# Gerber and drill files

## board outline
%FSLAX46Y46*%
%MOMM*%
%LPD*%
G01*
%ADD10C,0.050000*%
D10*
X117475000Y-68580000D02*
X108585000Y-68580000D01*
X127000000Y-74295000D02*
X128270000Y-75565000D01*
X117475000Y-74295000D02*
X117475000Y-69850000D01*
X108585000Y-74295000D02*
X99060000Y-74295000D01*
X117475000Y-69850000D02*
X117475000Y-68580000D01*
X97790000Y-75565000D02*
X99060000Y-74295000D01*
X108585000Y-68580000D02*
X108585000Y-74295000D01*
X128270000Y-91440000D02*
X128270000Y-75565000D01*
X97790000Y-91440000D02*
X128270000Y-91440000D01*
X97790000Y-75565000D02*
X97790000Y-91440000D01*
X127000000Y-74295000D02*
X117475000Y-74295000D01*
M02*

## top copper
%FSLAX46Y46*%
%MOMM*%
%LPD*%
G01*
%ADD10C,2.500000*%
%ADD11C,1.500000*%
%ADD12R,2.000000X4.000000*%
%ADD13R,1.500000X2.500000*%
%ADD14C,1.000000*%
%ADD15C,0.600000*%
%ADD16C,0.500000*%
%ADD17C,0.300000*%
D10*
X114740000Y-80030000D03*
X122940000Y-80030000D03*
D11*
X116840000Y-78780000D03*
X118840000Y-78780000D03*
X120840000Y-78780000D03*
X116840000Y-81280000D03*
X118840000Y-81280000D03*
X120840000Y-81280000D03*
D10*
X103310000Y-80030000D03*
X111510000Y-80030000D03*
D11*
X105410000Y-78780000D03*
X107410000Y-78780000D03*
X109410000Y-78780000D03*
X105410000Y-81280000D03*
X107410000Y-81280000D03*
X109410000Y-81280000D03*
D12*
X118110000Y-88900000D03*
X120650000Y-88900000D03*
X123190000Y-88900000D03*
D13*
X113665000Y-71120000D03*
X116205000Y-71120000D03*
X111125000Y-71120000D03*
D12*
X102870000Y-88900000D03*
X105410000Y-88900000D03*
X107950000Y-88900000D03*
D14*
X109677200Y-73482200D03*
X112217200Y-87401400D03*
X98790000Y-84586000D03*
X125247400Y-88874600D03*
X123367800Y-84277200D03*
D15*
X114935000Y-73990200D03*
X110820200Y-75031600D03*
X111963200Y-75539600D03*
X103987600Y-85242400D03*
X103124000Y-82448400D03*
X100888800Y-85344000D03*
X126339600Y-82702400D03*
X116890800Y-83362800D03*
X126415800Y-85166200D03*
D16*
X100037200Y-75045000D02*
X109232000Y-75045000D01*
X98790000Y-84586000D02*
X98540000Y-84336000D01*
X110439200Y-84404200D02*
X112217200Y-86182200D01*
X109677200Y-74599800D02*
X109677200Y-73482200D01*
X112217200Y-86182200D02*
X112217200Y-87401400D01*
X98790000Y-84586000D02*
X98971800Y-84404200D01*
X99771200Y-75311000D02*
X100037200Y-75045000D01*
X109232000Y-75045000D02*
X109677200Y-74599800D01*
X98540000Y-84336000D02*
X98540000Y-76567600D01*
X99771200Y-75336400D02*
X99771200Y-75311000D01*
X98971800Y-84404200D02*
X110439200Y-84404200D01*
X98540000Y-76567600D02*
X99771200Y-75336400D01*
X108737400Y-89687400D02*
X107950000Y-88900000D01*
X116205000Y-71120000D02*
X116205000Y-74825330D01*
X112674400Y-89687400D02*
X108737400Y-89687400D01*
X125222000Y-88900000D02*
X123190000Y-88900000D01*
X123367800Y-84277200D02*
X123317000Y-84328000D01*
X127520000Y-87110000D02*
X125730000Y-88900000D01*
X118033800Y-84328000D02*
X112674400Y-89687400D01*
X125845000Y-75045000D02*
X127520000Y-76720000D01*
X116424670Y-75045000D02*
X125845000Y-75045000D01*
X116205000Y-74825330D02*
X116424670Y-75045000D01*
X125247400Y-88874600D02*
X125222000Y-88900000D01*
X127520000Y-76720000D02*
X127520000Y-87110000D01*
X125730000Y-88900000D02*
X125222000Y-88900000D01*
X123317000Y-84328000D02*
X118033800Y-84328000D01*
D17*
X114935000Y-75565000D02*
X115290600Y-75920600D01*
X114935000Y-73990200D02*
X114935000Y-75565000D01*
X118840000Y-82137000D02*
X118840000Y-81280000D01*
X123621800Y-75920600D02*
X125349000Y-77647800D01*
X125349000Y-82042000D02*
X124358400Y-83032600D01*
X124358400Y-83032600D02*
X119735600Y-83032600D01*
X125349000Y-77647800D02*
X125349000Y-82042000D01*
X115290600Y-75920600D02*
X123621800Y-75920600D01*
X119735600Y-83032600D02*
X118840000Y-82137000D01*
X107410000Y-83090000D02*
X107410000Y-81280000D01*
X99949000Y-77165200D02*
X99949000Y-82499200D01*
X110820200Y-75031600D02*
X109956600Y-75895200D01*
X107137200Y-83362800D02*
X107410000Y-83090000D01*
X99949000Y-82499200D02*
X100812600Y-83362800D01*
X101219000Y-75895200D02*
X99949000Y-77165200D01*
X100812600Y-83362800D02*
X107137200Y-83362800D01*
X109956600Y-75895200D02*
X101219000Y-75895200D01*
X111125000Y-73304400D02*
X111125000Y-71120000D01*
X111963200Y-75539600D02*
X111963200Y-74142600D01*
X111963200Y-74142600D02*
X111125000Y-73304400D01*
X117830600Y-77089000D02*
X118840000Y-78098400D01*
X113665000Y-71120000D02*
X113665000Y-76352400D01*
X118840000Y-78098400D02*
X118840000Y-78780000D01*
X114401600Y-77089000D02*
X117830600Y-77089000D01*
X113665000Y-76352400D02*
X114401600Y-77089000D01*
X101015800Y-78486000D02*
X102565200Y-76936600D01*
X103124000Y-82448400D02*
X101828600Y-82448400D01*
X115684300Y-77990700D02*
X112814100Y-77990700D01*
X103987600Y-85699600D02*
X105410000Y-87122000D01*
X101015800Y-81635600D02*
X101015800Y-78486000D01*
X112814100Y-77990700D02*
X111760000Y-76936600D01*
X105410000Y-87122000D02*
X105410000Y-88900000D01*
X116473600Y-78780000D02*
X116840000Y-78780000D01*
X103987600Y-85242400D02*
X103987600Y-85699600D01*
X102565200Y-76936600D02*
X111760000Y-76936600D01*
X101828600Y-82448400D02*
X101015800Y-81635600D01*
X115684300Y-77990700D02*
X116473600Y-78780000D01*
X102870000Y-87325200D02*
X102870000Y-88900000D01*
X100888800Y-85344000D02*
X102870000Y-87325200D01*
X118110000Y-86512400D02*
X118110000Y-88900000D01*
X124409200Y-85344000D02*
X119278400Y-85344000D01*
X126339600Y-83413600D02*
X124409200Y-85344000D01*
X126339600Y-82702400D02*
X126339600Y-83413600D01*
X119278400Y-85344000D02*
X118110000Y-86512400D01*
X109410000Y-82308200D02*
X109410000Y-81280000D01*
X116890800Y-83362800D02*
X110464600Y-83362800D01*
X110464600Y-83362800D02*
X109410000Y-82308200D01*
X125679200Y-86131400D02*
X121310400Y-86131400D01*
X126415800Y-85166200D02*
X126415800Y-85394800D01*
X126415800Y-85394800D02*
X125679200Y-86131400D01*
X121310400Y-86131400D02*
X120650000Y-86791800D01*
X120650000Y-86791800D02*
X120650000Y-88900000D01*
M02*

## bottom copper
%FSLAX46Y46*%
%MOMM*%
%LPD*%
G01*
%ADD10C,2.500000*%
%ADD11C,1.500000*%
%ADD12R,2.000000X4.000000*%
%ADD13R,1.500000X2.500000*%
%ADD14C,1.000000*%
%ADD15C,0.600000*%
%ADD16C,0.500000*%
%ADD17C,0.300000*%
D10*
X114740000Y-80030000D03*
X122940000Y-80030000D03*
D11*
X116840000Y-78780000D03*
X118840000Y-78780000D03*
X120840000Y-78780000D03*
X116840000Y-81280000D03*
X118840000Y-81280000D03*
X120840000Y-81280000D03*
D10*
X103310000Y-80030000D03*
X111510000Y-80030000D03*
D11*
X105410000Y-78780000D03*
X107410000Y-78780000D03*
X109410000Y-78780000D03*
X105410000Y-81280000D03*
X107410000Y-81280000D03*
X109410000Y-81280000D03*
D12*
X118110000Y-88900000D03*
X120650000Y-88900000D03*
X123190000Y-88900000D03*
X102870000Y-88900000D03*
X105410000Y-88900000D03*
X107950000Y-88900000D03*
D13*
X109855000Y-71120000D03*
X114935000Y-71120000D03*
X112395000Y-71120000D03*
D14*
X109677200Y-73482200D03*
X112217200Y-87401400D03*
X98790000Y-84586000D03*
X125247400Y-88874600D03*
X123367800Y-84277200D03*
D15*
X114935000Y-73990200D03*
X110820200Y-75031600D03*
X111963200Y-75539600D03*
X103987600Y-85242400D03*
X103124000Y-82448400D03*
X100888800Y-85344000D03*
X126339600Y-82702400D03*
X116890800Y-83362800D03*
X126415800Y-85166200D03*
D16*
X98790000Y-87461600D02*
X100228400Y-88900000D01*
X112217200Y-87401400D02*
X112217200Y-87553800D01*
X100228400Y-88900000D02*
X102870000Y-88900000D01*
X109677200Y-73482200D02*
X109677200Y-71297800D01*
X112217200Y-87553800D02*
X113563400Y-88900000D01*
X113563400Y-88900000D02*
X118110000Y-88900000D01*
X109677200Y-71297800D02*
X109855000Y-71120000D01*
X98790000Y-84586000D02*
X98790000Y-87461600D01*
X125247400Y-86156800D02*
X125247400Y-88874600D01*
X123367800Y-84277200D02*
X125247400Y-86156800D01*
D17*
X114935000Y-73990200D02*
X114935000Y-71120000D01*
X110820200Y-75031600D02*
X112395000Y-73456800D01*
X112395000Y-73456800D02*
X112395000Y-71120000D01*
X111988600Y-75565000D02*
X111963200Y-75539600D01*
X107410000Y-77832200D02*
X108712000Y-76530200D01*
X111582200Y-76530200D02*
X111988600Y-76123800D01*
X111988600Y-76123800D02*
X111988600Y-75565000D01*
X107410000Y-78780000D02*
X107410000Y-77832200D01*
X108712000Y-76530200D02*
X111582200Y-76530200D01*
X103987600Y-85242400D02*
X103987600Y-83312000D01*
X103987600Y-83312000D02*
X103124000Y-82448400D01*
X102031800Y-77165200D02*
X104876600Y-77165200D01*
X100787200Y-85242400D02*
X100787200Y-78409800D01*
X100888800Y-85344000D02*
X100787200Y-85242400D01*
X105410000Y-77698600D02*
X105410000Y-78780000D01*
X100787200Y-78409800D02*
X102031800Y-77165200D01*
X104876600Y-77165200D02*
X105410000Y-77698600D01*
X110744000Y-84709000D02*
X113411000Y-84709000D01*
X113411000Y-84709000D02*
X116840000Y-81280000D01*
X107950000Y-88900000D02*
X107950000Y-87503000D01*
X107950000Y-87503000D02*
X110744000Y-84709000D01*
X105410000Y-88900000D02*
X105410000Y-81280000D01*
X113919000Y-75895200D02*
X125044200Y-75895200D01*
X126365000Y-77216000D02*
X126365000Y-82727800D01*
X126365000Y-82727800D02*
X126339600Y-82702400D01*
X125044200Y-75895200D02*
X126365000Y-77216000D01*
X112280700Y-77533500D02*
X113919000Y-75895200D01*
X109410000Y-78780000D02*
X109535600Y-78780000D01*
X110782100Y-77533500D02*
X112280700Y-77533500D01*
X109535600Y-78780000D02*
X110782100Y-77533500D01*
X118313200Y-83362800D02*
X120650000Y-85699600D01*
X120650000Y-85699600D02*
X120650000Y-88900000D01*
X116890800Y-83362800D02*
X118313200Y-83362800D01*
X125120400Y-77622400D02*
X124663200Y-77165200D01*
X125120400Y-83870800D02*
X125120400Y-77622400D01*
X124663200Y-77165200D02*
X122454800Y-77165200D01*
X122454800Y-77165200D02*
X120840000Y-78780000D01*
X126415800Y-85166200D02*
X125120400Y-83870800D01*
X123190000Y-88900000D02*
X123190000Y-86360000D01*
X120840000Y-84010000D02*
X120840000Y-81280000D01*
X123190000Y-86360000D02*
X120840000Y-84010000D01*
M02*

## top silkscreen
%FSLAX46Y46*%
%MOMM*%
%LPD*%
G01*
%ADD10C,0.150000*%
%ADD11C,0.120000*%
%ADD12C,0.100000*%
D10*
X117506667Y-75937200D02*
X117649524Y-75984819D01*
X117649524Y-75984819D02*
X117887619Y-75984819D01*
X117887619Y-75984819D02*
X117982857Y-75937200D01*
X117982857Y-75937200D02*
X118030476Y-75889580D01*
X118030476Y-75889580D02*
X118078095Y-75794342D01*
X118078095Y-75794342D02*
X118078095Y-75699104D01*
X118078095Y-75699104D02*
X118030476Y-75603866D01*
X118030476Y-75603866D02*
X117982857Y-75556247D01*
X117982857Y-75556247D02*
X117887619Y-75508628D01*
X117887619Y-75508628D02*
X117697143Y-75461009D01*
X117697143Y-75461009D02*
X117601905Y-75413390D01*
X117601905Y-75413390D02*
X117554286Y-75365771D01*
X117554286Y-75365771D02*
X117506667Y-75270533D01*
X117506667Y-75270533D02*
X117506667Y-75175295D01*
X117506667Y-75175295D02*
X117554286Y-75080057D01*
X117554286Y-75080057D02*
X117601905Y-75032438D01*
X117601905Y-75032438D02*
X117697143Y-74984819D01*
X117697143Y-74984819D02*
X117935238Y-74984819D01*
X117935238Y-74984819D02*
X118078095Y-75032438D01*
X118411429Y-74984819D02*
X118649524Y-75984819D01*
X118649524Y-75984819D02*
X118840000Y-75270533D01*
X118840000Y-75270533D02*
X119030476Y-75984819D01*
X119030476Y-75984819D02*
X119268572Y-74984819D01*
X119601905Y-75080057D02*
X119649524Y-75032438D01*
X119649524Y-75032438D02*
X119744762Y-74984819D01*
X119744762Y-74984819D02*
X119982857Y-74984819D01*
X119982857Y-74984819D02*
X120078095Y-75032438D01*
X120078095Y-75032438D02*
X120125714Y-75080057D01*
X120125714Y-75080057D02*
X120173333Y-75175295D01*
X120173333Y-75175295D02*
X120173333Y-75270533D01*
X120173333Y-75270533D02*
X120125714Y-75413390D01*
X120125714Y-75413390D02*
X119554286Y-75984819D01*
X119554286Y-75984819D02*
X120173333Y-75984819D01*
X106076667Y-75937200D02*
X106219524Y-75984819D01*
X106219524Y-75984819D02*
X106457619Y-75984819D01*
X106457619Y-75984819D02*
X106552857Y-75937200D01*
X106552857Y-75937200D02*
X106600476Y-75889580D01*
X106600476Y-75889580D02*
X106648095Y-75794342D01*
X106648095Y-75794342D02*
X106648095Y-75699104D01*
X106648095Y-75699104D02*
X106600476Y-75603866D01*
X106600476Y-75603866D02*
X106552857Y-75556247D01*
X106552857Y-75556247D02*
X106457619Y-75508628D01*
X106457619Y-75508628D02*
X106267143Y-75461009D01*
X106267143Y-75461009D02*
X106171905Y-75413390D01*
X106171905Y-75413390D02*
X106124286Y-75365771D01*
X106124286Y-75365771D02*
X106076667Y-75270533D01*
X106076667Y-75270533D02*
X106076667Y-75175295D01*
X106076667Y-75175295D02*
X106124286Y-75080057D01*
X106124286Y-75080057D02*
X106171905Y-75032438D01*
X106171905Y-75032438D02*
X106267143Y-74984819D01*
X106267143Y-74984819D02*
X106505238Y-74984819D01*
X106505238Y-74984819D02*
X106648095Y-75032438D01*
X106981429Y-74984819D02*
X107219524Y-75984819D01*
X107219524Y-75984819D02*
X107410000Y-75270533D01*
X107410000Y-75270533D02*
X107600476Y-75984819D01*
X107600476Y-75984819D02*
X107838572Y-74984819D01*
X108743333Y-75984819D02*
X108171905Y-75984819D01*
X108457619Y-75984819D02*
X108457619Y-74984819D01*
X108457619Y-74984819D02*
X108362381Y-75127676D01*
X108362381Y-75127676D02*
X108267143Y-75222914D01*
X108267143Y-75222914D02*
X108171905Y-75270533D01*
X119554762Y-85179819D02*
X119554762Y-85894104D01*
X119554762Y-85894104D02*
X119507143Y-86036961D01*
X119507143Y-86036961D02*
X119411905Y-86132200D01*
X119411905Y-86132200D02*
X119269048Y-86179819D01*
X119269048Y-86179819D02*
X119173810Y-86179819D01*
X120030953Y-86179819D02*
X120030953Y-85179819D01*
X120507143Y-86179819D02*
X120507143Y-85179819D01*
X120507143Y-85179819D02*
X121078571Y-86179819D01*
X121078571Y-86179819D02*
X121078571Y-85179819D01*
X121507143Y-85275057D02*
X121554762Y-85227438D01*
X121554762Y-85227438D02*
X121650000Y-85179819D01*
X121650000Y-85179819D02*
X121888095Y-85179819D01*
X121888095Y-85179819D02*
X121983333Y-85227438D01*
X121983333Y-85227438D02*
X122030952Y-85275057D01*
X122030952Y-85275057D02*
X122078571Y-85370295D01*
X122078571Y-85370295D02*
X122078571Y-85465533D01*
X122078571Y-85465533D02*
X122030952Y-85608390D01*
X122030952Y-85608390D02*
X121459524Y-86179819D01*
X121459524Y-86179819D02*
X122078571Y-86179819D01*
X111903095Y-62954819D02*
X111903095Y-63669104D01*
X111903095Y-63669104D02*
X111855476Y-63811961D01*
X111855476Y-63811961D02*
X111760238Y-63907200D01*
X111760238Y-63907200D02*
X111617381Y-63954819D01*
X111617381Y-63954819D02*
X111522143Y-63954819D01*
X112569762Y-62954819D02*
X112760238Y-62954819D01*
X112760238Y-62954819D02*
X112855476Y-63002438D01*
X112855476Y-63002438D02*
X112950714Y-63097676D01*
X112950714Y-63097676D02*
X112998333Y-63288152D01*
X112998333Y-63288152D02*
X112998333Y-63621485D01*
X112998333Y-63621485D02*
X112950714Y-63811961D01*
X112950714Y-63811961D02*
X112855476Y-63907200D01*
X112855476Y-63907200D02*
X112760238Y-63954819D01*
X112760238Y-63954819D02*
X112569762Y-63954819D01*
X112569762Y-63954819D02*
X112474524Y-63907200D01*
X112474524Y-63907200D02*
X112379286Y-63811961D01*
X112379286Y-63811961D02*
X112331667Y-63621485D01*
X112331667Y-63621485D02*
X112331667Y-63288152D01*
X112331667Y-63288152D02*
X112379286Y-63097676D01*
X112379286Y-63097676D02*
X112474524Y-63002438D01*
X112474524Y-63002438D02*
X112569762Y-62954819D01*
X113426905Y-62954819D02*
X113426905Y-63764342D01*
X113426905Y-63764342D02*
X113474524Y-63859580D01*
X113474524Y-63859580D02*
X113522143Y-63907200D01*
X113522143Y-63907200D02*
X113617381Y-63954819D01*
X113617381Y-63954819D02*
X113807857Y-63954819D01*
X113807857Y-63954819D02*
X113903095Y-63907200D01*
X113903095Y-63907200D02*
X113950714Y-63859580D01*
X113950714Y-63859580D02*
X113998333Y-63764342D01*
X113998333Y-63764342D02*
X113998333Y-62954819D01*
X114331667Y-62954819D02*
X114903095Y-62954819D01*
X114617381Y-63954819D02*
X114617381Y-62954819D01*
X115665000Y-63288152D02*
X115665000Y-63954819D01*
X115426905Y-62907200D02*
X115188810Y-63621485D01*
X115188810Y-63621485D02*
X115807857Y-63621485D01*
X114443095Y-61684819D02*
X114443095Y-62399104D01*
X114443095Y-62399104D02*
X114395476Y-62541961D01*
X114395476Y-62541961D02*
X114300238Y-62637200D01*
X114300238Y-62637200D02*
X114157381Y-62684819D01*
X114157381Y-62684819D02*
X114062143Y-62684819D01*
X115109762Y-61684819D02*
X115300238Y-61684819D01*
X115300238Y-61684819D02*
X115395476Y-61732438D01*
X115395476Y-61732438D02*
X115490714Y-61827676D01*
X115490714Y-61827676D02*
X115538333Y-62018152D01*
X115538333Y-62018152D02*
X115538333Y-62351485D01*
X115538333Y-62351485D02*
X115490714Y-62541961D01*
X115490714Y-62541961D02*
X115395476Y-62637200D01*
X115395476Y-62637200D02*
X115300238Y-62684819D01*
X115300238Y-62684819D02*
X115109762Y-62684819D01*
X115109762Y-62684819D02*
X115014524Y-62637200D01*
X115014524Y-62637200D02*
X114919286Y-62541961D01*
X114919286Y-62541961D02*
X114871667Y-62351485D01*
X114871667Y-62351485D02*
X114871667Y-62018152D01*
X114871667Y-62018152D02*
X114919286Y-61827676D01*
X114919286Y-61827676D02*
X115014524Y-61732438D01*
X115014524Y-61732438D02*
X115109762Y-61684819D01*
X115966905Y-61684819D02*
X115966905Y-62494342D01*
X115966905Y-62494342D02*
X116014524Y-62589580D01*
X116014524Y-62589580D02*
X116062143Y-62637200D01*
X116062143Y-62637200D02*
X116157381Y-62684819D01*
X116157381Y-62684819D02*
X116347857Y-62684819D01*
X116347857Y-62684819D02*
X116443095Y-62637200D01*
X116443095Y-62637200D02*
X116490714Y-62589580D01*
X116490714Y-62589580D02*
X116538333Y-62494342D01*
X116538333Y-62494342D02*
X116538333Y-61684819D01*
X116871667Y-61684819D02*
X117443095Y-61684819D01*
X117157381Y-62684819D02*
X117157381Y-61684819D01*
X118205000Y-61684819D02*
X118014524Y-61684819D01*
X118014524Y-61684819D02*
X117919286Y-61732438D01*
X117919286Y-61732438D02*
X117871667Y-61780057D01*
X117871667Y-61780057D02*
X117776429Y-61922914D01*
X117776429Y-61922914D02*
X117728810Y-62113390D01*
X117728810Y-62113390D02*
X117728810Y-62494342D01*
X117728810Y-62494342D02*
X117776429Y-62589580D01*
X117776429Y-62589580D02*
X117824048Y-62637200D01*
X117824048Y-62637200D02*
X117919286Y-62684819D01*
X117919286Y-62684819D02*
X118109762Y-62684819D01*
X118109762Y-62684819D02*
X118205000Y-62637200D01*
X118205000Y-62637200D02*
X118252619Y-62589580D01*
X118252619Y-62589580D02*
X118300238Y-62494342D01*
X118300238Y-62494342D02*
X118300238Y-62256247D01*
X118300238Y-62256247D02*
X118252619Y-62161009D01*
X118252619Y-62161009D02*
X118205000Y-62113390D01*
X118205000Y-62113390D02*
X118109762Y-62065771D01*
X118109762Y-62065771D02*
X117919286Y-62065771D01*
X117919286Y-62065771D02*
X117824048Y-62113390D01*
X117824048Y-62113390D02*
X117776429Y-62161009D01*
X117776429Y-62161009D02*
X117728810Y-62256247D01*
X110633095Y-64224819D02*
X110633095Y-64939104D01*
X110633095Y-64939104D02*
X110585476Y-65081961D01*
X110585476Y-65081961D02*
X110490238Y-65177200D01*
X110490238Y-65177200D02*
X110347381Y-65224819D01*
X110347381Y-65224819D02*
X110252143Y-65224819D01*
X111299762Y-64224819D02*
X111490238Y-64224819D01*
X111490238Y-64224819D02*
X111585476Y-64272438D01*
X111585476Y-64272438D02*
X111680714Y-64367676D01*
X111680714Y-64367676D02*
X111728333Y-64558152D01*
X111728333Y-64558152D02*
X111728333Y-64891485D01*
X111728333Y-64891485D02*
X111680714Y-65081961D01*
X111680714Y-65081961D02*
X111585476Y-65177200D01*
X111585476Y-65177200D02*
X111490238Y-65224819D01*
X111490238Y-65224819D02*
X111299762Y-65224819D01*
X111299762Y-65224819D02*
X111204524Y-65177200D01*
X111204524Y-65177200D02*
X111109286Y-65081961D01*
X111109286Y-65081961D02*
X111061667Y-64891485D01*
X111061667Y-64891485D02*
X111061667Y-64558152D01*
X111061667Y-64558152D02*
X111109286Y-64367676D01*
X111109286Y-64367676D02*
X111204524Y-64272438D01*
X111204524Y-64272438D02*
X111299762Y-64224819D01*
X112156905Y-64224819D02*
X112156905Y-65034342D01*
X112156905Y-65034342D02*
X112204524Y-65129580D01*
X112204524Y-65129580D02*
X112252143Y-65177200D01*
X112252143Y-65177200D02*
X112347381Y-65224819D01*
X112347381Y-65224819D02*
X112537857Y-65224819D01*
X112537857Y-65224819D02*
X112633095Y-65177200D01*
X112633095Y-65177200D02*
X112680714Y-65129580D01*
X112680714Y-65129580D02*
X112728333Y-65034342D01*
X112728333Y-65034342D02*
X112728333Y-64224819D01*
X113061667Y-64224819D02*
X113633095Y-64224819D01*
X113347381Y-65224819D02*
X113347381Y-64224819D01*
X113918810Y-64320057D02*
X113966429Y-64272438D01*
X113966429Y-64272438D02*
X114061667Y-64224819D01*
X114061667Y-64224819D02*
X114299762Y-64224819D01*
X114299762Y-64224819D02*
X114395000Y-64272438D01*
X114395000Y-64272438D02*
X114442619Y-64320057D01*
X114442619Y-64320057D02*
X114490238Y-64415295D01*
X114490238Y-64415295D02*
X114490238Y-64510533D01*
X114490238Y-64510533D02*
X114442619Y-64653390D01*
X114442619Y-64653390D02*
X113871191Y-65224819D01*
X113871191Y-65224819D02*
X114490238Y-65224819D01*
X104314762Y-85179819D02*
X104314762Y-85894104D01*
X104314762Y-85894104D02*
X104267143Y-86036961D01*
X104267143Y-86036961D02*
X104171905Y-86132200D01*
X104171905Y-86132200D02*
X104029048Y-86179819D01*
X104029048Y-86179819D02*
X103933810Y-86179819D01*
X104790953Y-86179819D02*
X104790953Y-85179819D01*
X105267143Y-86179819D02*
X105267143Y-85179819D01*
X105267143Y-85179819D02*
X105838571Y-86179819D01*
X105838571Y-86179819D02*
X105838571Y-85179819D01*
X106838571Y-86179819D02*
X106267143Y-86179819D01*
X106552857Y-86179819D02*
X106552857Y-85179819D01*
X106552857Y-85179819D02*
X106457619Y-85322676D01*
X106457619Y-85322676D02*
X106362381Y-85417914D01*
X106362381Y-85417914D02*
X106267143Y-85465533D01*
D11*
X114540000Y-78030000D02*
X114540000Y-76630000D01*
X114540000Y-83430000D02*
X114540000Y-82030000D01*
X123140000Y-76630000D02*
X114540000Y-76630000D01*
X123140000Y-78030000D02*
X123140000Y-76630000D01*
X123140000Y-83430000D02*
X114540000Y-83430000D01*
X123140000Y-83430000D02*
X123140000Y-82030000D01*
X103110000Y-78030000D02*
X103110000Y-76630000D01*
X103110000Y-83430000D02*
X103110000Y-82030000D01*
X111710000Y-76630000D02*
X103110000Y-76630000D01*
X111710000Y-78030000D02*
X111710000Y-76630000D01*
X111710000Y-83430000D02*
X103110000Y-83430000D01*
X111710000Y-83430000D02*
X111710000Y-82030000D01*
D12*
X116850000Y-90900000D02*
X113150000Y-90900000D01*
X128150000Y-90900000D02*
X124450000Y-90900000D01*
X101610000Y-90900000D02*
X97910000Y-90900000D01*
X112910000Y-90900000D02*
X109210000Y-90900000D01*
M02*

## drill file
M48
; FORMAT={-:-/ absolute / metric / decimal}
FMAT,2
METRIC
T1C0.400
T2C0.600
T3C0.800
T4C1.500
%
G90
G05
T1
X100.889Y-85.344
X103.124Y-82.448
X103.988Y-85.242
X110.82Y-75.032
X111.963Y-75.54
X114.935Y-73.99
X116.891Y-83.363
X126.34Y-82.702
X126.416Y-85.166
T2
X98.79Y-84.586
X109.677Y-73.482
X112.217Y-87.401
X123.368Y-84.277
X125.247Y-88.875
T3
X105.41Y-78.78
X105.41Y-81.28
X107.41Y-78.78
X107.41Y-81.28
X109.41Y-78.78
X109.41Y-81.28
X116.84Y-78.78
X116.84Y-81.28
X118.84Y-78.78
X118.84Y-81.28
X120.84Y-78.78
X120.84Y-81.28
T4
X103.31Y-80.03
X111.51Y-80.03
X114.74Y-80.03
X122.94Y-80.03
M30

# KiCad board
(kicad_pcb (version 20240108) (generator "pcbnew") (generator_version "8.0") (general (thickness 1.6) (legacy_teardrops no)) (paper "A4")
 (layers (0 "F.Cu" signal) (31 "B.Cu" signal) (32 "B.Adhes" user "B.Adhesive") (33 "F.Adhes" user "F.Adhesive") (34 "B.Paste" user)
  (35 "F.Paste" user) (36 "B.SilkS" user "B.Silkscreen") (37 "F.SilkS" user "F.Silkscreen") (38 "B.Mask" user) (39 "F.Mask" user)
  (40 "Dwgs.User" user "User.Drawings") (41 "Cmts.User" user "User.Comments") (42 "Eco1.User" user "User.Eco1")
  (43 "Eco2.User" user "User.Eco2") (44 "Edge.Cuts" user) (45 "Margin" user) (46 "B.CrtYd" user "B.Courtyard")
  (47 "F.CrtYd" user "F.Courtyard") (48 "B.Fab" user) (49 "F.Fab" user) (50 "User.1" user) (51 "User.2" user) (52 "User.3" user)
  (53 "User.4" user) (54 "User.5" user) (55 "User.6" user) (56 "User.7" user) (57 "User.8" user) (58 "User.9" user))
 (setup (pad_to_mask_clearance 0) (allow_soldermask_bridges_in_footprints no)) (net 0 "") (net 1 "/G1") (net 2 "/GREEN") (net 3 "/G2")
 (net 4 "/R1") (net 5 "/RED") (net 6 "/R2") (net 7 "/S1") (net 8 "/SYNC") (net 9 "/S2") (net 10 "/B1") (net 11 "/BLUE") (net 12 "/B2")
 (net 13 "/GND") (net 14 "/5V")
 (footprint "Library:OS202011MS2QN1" (layer "F.Cu") (at 118.84 80.03)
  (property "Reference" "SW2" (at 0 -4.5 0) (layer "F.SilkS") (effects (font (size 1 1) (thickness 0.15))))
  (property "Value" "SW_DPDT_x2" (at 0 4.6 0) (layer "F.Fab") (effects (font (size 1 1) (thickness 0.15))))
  (fp_line (start -4.3 -2) (end -4.3 -3.4) (stroke (width 0.12) (type solid)) (layer "F.SilkS"))
  (fp_line (start -4.3 3.4) (end -4.3 2) (stroke (width 0.12) (type solid)) (layer "F.SilkS"))
  (fp_line (start 4.3 -3.4) (end -4.3 -3.4) (stroke (width 0.12) (type solid)) (layer "F.SilkS"))
  (fp_line (start 4.3 -2) (end 4.3 -3.4) (stroke (width 0.12) (type solid)) (layer "F.SilkS"))
  (fp_line (start 4.3 3.4) (end -4.3 3.4) (stroke (width 0.12) (type solid)) (layer "F.SilkS"))
  (fp_line (start 4.3 3.4) (end 4.3 2) (stroke (width 0.12) (type solid)) (layer "F.SilkS"))
  (pad "" thru_hole circle (at -4.1 0) (size 2.5 2.5) (drill 1.5) (layers "*.Cu" "*.Mask") (remove_unused_layers no))
  (pad "" thru_hole circle (at 4.1 0) (size 2.5 2.5) (drill 1.5) (layers "*.Cu" "*.Mask") (remove_unused_layers no))
  (pad "1" thru_hole circle (at -2 -1.25) (size 1.5 1.5) (drill 0.8) (layers "*.Cu" "*.Mask") (remove_unused_layers no) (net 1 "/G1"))
  (pad "2" thru_hole circle (at 0 -1.25) (size 1.5 1.5) (drill 0.8) (layers "*.Cu" "*.Mask") (remove_unused_layers no) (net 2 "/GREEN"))
  (pad "3" thru_hole circle (at 2 -1.25) (size 1.5 1.5) (drill 0.8) (layers "*.Cu" "*.Mask") (remove_unused_layers no) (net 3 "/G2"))
  (pad "4" thru_hole circle (at -2 1.25) (size 1.5 1.5) (drill 0.8) (layers "*.Cu" "*.Mask") (remove_unused_layers no) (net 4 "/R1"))
  (pad "5" thru_hole circle (at 0 1.25) (size 1.5 1.5) (drill 0.8) (layers "*.Cu" "*.Mask") (remove_unused_layers no) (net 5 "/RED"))
  (pad "6" thru_hole circle (at 2 1.25) (size 1.5 1.5) (drill 0.8) (layers "*.Cu" "*.Mask") (remove_unused_layers no) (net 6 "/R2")))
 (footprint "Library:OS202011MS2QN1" (layer "F.Cu") (at 107.41 80.03)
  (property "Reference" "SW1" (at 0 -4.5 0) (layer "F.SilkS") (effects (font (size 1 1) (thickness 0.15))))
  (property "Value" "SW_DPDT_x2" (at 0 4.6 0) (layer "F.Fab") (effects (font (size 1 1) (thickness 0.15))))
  (fp_line (start -4.3 -2) (end -4.3 -3.4) (stroke (width 0.12) (type solid)) (layer "F.SilkS"))
  (fp_line (start -4.3 3.4) (end -4.3 2) (stroke (width 0.12) (type solid)) (layer "F.SilkS"))
  (fp_line (start 4.3 -3.4) (end -4.3 -3.4) (stroke (width 0.12) (type solid)) (layer "F.SilkS"))
  (fp_line (start 4.3 -2) (end 4.3 -3.4) (stroke (width 0.12) (type solid)) (layer "F.SilkS"))
  (fp_line (start 4.3 3.4) (end -4.3 3.4) (stroke (width 0.12) (type solid)) (layer "F.SilkS"))
  (fp_line (start 4.3 3.4) (end 4.3 2) (stroke (width 0.12) (type solid)) (layer "F.SilkS"))
  (pad "" thru_hole circle (at -4.1 0) (size 2.5 2.5) (drill 1.5) (layers "*.Cu" "*.Mask") (remove_unused_layers no))
  (pad "" thru_hole circle (at 4.1 0) (size 2.5 2.5) (drill 1.5) (layers "*.Cu" "*.Mask") (remove_unused_layers no))
  (pad "1" thru_hole circle (at -2 -1.25) (size 1.5 1.5) (drill 0.8) (layers "*.Cu" "*.Mask") (remove_unused_layers no) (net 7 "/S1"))
  (pad "2" thru_hole circle (at 0 -1.25) (size 1.5 1.5) (drill 0.8) (layers "*.Cu" "*.Mask") (remove_unused_layers no) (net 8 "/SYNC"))
  (pad "3" thru_hole circle (at 2 -1.25) (size 1.5 1.5) (drill 0.8) (layers "*.Cu" "*.Mask") (remove_unused_layers no) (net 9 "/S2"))
  (pad "4" thru_hole circle (at -2 1.25) (size 1.5 1.5) (drill 0.8) (layers "*.Cu" "*.Mask") (remove_unused_layers no) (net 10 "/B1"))
  (pad "5" thru_hole circle (at 0 1.25) (size 1.5 1.5) (drill 0.8) (layers "*.Cu" "*.Mask") (remove_unused_layers no) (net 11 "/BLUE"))
  (pad "6" thru_hole circle (at 2 1.25) (size 1.5 1.5) (drill 0.8) (layers "*.Cu" "*.Mask") (remove_unused_layers no) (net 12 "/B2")))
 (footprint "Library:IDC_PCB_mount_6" (layer "F.Cu") (at 120.65 88.9)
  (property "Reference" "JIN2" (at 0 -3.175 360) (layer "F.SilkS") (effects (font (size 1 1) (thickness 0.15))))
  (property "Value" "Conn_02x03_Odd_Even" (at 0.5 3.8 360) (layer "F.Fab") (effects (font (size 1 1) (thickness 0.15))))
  (fp_line (start -3.8 2) (end -7.5 2) (stroke (width 0.1) (type default)) (layer "F.SilkS"))
  (fp_line (start 7.5 2) (end 3.8 2) (stroke (width 0.1) (type default)) (layer "F.SilkS"))
  (pad "1" smd rect (at -2.54 0) (size 2 4) (layers "B.Cu" "B.Mask") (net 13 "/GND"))
  (pad "2" smd rect (at -2.54 0) (size 2 4) (layers "F.Cu" "F.Mask") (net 9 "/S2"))
  (pad "3" smd rect (at 0 0) (size 2 4) (layers "B.Cu" "B.Mask") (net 12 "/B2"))
  (pad "4" smd rect (at 0 0) (size 2 4) (layers "F.Cu" "F.Mask") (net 3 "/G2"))
  (pad "5" smd rect (at 2.54 0) (size 2 4) (layers "B.Cu" "B.Mask") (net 6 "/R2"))
  (pad "6" smd rect (at 2.54 0) (size 2 4) (layers "F.Cu" "F.Mask") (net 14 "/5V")))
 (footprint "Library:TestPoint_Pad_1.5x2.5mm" (layer "F.Cu") (at 113.665 71.12)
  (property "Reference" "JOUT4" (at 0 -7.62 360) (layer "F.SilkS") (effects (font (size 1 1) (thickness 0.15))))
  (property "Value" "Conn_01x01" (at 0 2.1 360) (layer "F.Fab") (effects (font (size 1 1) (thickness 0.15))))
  (pad "1" smd rect (at 0 0) (size 1.5 2.5) (layers "F.Cu" "F.Mask") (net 2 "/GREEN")))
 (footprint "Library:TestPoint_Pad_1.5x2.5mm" (layer "F.Cu") (at 116.205 71.12)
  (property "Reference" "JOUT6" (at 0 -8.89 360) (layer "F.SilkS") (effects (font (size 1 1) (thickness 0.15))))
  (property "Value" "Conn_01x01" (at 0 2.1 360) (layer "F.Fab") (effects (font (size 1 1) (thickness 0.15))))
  (pad "1" smd rect (at 0 0) (size 1.5 2.5) (layers "F.Cu" "F.Mask") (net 14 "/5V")))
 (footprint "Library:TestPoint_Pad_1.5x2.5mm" (layer "F.Cu") (at 111.125 71.12)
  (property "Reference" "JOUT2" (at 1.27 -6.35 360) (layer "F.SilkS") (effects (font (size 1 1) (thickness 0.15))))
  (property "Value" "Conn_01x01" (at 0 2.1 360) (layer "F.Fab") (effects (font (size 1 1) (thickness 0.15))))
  (pad "1" smd rect (at 0 0) (size 1.5 2.5) (layers "F.Cu" "F.Mask") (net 8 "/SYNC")))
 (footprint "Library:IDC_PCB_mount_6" (layer "F.Cu") (at 105.41 88.9)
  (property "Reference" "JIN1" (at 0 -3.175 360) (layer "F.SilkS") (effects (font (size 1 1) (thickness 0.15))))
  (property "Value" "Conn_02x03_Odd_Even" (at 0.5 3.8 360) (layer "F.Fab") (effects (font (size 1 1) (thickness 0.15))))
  (fp_line (start -3.8 2) (end -7.5 2) (stroke (width 0.1) (type default)) (layer "F.SilkS"))
  (fp_line (start 7.5 2) (end 3.8 2) (stroke (width 0.1) (type default)) (layer "F.SilkS"))
  (pad "1" smd rect (at -2.54 0) (size 2 4) (layers "B.Cu" "B.Mask") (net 13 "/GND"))
  (pad "2" smd rect (at -2.54 0) (size 2 4) (layers "F.Cu" "F.Mask") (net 7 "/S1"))
  (pad "3" smd rect (at 0 0) (size 2 4) (layers "B.Cu" "B.Mask") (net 10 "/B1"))
  (pad "4" smd rect (at 0 0) (size 2 4) (layers "F.Cu" "F.Mask") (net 1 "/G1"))
  (pad "5" smd rect (at 2.54 0) (size 2 4) (layers "B.Cu" "B.Mask") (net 4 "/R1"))
  (pad "6" smd rect (at 2.54 0) (size 2 4) (layers "F.Cu" "F.Mask") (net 14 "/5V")))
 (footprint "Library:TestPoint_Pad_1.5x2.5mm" (layer "B.Cu") (at 109.855 71.12 180)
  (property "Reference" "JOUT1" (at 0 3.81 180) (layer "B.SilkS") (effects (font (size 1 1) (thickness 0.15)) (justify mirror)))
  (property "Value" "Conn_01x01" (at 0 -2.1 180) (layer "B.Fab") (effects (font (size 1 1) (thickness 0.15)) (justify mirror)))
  (pad "1" smd rect (at 0 0 180) (size 1.5 2.5) (layers "B.Cu" "B.Mask") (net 13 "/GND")))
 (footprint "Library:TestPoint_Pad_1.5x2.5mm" (layer "B.Cu") (at 114.935 71.12 180)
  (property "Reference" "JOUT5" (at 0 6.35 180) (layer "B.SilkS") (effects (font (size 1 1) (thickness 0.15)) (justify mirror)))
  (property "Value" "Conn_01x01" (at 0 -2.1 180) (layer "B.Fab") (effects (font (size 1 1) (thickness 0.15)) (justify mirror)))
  (pad "1" smd rect (at 0 0 180) (size 1.5 2.5) (layers "B.Cu" "B.Mask") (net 5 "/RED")))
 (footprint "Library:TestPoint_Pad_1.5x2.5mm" (layer "B.Cu") (at 112.395 71.12 180)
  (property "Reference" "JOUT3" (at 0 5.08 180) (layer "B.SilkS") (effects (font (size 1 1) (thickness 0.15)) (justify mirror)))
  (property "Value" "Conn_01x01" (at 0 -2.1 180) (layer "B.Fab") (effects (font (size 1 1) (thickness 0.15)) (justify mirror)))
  (pad "1" smd rect (at 0 0 180) (size 1.5 2.5) (layers "B.Cu" "B.Mask") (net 11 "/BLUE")))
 (gr_line (start 117.475 68.58) (end 108.585 68.58) (stroke (width 0.05) (type default)) (layer "Edge.Cuts"))
 (gr_line (start 127 74.295) (end 128.27 75.565) (stroke (width 0.05) (type default)) (layer "Edge.Cuts"))
 (gr_line (start 117.475 74.295) (end 117.475 69.85) (stroke (width 0.05) (type default)) (layer "Edge.Cuts"))
 (gr_line (start 108.585 74.295) (end 99.06 74.295) (stroke (width 0.05) (type default)) (layer "Edge.Cuts"))
 (gr_line (start 117.475 69.85) (end 117.475 68.58) (stroke (width 0.05) (type default)) (layer "Edge.Cuts"))
 (gr_line (start 97.79 75.565) (end 99.06 74.295) (stroke (width 0.05) (type default)) (layer "Edge.Cuts"))
 (gr_line (start 108.585 68.58) (end 108.585 74.295) (stroke (width 0.05) (type default)) (layer "Edge.Cuts"))
 (gr_line (start 128.27 91.44) (end 128.27 75.565) (stroke (width 0.05) (type default)) (layer "Edge.Cuts"))
 (gr_line (start 97.79 91.44) (end 128.27 91.44) (stroke (width 0.05) (type default)) (layer "Edge.Cuts"))
 (gr_line (start 97.79 75.565) (end 97.79 91.44) (stroke (width 0.05) (type default)) (layer "Edge.Cuts"))
 (gr_line (start 127 74.295) (end 117.475 74.295) (stroke (width 0.05) (type default)) (layer "Edge.Cuts"))
 (segment (start 100.0372 75.045) (end 109.232 75.045) (width 0.5) (layer "F.Cu") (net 13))
 (segment (start 98.79 84.586) (end 98.54 84.336) (width 0.5) (layer "F.Cu") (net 13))
 (segment (start 110.4392 84.4042) (end 112.2172 86.1822) (width 0.5) (layer "F.Cu") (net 13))
 (segment (start 109.6772 74.5998) (end 109.6772 73.4822) (width 0.5) (layer "F.Cu") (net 13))
 (segment (start 112.2172 86.1822) (end 112.2172 87.4014) (width 0.5) (layer "F.Cu") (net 13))
 (segment (start 98.79 84.586) (end 98.9718 84.4042) (width 0.5) (layer "F.Cu") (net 13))
 (segment (start 99.7712 75.311) (end 100.0372 75.045) (width 0.5) (layer "F.Cu") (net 13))
 (segment (start 109.232 75.045) (end 109.6772 74.5998) (width 0.5) (layer "F.Cu") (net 13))
 (segment (start 98.54 84.336) (end 98.54 76.5676) (width 0.5) (layer "F.Cu") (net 13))
 (segment (start 99.7712 75.3364) (end 99.7712 75.311) (width 0.5) (layer "F.Cu") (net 13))
 (segment (start 98.9718 84.4042) (end 110.4392 84.4042) (width 0.5) (layer "F.Cu") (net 13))
 (segment (start 98.54 76.5676) (end 99.7712 75.3364) (width 0.5) (layer "F.Cu") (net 13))
 (via (at 109.6772 73.4822) (size 1) (drill 0.6) (layers "F.Cu" "B.Cu") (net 13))
 (via (at 112.2172 87.4014) (size 1) (drill 0.6) (layers "F.Cu" "B.Cu") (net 13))
 (via (at 98.79 84.586) (size 1) (drill 0.6) (layers "F.Cu" "B.Cu") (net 13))
 (segment (start 98.79 87.4616) (end 100.2284 88.9) (width 0.5) (layer "B.Cu") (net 13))
 (segment (start 112.2172 87.4014) (end 112.2172 87.5538) (width 0.5) (layer "B.Cu") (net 13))
 (segment (start 100.2284 88.9) (end 102.87 88.9) (width 0.5) (layer "B.Cu") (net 13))
 (segment (start 109.6772 73.4822) (end 109.6772 71.2978) (width 0.5) (layer "B.Cu") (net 13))
 (segment (start 112.2172 87.5538) (end 113.5634 88.9) (width 0.5) (layer "B.Cu") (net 13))
 (segment (start 113.5634 88.9) (end 118.11 88.9) (width 0.5) (layer "B.Cu") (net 13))
 (segment (start 109.6772 71.2978) (end 109.855 71.12) (width 0.5) (layer "B.Cu") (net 13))
 (segment (start 98.79 84.586) (end 98.79 87.4616) (width 0.5) (layer "B.Cu") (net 13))
 (segment (start 108.7374 89.6874) (end 107.95 88.9) (width 0.5) (layer "F.Cu") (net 14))
 (segment (start 116.205 71.12) (end 116.205 74.82533) (width 0.5) (layer "F.Cu") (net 14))
 (segment (start 112.6744 89.6874) (end 108.7374 89.6874) (width 0.5) (layer "F.Cu") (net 14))
 (segment (start 125.222 88.9) (end 123.19 88.9) (width 0.5) (layer "F.Cu") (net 14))
 (segment (start 123.3678 84.2772) (end 123.317 84.328) (width 0.5) (layer "F.Cu") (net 14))
 (segment (start 127.52 87.11) (end 125.73 88.9) (width 0.5) (layer "F.Cu") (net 14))
 (segment (start 118.0338 84.328) (end 112.6744 89.6874) (width 0.5) (layer "F.Cu") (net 14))
 (segment (start 125.845 75.045) (end 127.52 76.72) (width 0.5) (layer "F.Cu") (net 14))
 (segment (start 116.42467 75.045) (end 125.845 75.045) (width 0.5) (layer "F.Cu") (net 14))
 (segment (start 116.205 74.82533) (end 116.42467 75.045) (width 0.5) (layer "F.Cu") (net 14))
 (segment (start 125.2474 88.8746) (end 125.222 88.9) (width 0.5) (layer "F.Cu") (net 14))
 (segment (start 127.52 76.72) (end 127.52 87.11) (width 0.5) (layer "F.Cu") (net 14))
 (segment (start 125.73 88.9) (end 125.222 88.9) (width 0.5) (layer "F.Cu") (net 14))
 (segment (start 123.317 84.328) (end 118.0338 84.328) (width 0.5) (layer "F.Cu") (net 14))
 (via (at 125.2474 88.8746) (size 1) (drill 0.6) (layers "F.Cu" "B.Cu") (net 14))
 (via (at 123.3678 84.2772) (size 1) (drill 0.6) (layers "F.Cu" "B.Cu") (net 14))
 (segment (start 125.2474 86.1568) (end 125.2474 88.8746) (width 0.5) (layer "B.Cu") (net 14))
 (segment (start 123.3678 84.2772) (end 125.2474 86.1568) (width 0.5) (layer "B.Cu") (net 14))
 (segment (start 114.935 75.565) (end 115.2906 75.9206) (width 0.3) (layer "F.Cu") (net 5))
 (segment (start 114.935 73.9902) (end 114.935 75.565) (width 0.3) (layer "F.Cu") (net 5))
 (segment (start 118.84 82.137) (end 118.84 81.28) (width 0.3) (layer "F.Cu") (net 5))
 (segment (start 123.6218 75.9206) (end 125.349 77.6478) (width 0.3) (layer "F.Cu") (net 5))
 (segment (start 125.349 82.042) (end 124.3584 83.0326) (width 0.3) (layer "F.Cu") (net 5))
 (segment (start 124.3584 83.0326) (end 119.7356 83.0326) (width 0.3) (layer "F.Cu") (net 5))
 (segment (start 125.349 77.6478) (end 125.349 82.042) (width 0.3) (layer "F.Cu") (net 5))
 (segment (start 115.2906 75.9206) (end 123.6218 75.9206) (width 0.3) (layer "F.Cu") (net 5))
 (segment (start 119.7356 83.0326) (end 118.84 82.137) (width 0.3) (layer "F.Cu") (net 5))
 (via (at 114.935 73.9902) (size 0.6) (drill 0.4) (layers "F.Cu" "B.Cu") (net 5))
 (segment (start 114.935 73.9902) (end 114.935 71.12) (width 0.3) (layer "B.Cu") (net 5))
 (segment (start 107.41 83.09) (end 107.41 81.28) (width 0.3) (layer "F.Cu") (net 11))
 (segment (start 99.949 77.1652) (end 99.949 82.4992) (width 0.3) (layer "F.Cu") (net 11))
 (segment (start 110.8202 75.0316) (end 109.9566 75.8952) (width 0.3) (layer "F.Cu") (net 11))
 (segment (start 107.1372 83.3628) (end 107.41 83.09) (width 0.3) (layer "F.Cu") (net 11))
 (segment (start 99.949 82.4992) (end 100.8126 83.3628) (width 0.3) (layer "F.Cu") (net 11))
 (segment (start 101.219 75.8952) (end 99.949 77.1652) (width 0.3) (layer "F.Cu") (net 11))
 (segment (start 100.8126 83.3628) (end 107.1372 83.3628) (width 0.3) (layer "F.Cu") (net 11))
 (segment (start 109.9566 75.8952) (end 101.219 75.8952) (width 0.3) (layer "F.Cu") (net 11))
 (via (at 110.8202 75.0316) (size 0.6) (drill 0.4) (layers "F.Cu" "B.Cu") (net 11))
 (segment (start 110.8202 75.0316) (end 112.395 73.4568) (width 0.3) (layer "B.Cu") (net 11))
 (segment (start 112.395 73.4568) (end 112.395 71.12) (width 0.3) (layer "B.Cu") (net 11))
 (segment (start 111.125 73.3044) (end 111.125 71.12) (width 0.3) (layer "F.Cu") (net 8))
 (segment (start 111.9632 75.5396) (end 111.9632 74.1426) (width 0.3) (layer "F.Cu") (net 8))
 (segment (start 111.9632 74.1426) (end 111.125 73.3044) (width 0.3) (layer "F.Cu") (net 8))
 (via (at 111.9632 75.5396) (size 0.6) (drill 0.4) (layers "F.Cu" "B.Cu") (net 8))
 (segment (start 111.9886 75.565) (end 111.9632 75.5396) (width 0.3) (layer "B.Cu") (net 8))
 (segment (start 107.41 77.8322) (end 108.712 76.5302) (width 0.3) (layer "B.Cu") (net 8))
 (segment (start 111.5822 76.5302) (end 111.9886 76.1238) (width 0.3) (layer "B.Cu") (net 8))
 (segment (start 111.9886 76.1238) (end 111.9886 75.565) (width 0.3) (layer "B.Cu") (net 8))
 (segment (start 107.41 78.78) (end 107.41 77.8322) (width 0.3) (layer "B.Cu") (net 8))
 (segment (start 108.712 76.5302) (end 111.5822 76.5302) (width 0.3) (layer "B.Cu") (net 8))
 (segment (start 117.8306 77.089) (end 118.84 78.0984) (width 0.3) (layer "F.Cu") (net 2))
 (segment (start 113.665 71.12) (end 113.665 76.3524) (width 0.3) (layer "F.Cu") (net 2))
 (segment (start 118.84 78.0984) (end 118.84 78.78) (width 0.3) (layer "F.Cu") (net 2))
 (segment (start 114.4016 77.089) (end 117.8306 77.089) (width 0.3) (layer "F.Cu") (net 2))
 (segment (start 113.665 76.3524) (end 114.4016 77.089) (width 0.3) (layer "F.Cu") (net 2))
 (segment (start 101.0158 78.486) (end 102.5652 76.9366) (width 0.3) (layer "F.Cu") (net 1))
 (segment (start 103.124 82.4484) (end 101.8286 82.4484) (width 0.3) (layer "F.Cu") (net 1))
 (segment (start 115.6843 77.9907) (end 112.8141 77.9907) (width 0.3) (layer "F.Cu") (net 1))
 (segment (start 103.9876 85.6996) (end 105.41 87.122) (width 0.3) (layer "F.Cu") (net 1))
 (segment (start 101.0158 81.6356) (end 101.0158 78.486) (width 0.3) (layer "F.Cu") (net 1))
 (segment (start 112.8141 77.9907) (end 111.76 76.9366) (width 0.3) (layer "F.Cu") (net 1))
 (segment (start 105.41 87.122) (end 105.41 88.9) (width 0.3) (layer "F.Cu") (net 1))
 (segment (start 116.4736 78.78) (end 116.84 78.78) (width 0.3) (layer "F.Cu") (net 1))
 (segment (start 103.9876 85.2424) (end 103.9876 85.6996) (width 0.3) (layer "F.Cu") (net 1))
 (segment (start 102.5652 76.9366) (end 111.76 76.9366) (width 0.3) (layer "F.Cu") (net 1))
 (segment (start 101.8286 82.4484) (end 101.0158 81.6356) (width 0.3) (layer "F.Cu") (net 1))
 (segment (start 115.6843 77.9907) (end 116.4736 78.78) (width 0.3) (layer "F.Cu") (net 1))
 (via (at 103.9876 85.2424) (size 0.6) (drill 0.4) (layers "F.Cu" "B.Cu") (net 1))
 (via (at 103.124 82.4484) (size 0.6) (drill 0.4) (layers "F.Cu" "B.Cu") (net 1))
 (segment (start 103.9876 85.2424) (end 103.9876 83.312) (width 0.3) (layer "B.Cu") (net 1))
 (segment (start 103.9876 83.312) (end 103.124 82.4484) (width 0.3) (layer "B.Cu") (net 1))
 (segment (start 102.87 87.3252) (end 102.87 88.9) (width 0.3) (layer "F.Cu") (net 7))
 (segment (start 100.8888 85.344) (end 102.87 87.3252) (width 0.3) (layer "F.Cu") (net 7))
 (via (at 100.8888 85.344) (size 0.6) (drill 0.4) (layers "F.Cu" "B.Cu") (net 7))
 (segment (start 102.0318 77.1652) (end 104.8766 77.1652) (width 0.3) (layer "B.Cu") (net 7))
 (segment (start 100.7872 85.2424) (end 100.7872 78.4098) (width 0.3) (layer "B.Cu") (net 7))
 (segment (start 100.8888 85.344) (end 100.7872 85.2424) (width 0.3) (layer "B.Cu") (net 7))
 (segment (start 105.41 77.6986) (end 105.41 78.78) (width 0.3) (layer "B.Cu") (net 7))
 (segment (start 100.7872 78.4098) (end 102.0318 77.1652) (width 0.3) (layer "B.Cu") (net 7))
 (segment (start 104.8766 77.1652) (end 105.41 77.6986) (width 0.3) (layer "B.Cu") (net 7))
 (segment (start 110.744 84.709) (end 113.411 84.709) (width 0.3) (layer "B.Cu") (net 4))
 (segment (start 113.411 84.709) (end 116.84 81.28) (width 0.3) (layer "B.Cu") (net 4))
 (segment (start 107.95 88.9) (end 107.95 87.503) (width 0.3) (layer "B.Cu") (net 4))
 (segment (start 107.95 87.503) (end 110.744 84.709) (width 0.3) (layer "B.Cu") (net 4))
 (segment (start 105.41 88.9) (end 105.41 81.28) (width 0.3) (layer "B.Cu") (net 10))
 (segment (start 118.11 86.5124) (end 118.11 88.9) (width 0.3) (layer "F.Cu") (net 9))
 (segment (start 124.4092 85.344) (end 119.2784 85.344) (width 0.3) (layer "F.Cu") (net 9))
 (segment (start 126.3396 83.4136) (end 124.4092 85.344) (width 0.3) (layer "F.Cu") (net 9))
 (segment (start 126.3396 82.7024) (end 126.3396 83.4136) (width 0.3) (layer "F.Cu") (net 9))
 (segment (start 119.2784 85.344) (end 118.11 86.5124) (width 0.3) (layer "F.Cu") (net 9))
 (via (at 126.3396 82.7024) (size 0.6) (drill 0.4) (layers "F.Cu" "B.Cu") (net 9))
 (segment (start 113.919 75.8952) (end 125.0442 75.8952) (width 0.3) (layer "B.Cu") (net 9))
 (segment (start 126.365 77.216) (end 126.365 82.7278) (width 0.3) (layer "B.Cu") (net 9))
 (segment (start 126.365 82.7278) (end 126.3396 82.7024) (width 0.3) (layer "B.Cu") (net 9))
 (segment (start 125.0442 75.8952) (end 126.365 77.216) (width 0.3) (layer "B.Cu") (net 9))
 (segment (start 112.2807 77.5335) (end 113.919 75.8952) (width 0.3) (layer "B.Cu") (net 9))
 (segment (start 109.41 78.78) (end 109.5356 78.78) (width 0.3) (layer "B.Cu") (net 9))
 (segment (start 110.7821 77.5335) (end 112.2807 77.5335) (width 0.3) (layer "B.Cu") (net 9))
 (segment (start 109.5356 78.78) (end 110.7821 77.5335) (width 0.3) (layer "B.Cu") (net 9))
 (segment (start 109.41 82.3082) (end 109.41 81.28) (width 0.3) (layer "F.Cu") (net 12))
 (segment (start 116.8908 83.3628) (end 110.4646 83.3628) (width 0.3) (layer "F.Cu") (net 12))
 (segment (start 110.4646 83.3628) (end 109.41 82.3082) (width 0.3) (layer "F.Cu") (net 12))
 (via (at 116.8908 83.3628) (size 0.6) (drill 0.4) (layers "F.Cu" "B.Cu") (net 12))
 (segment (start 118.3132 83.3628) (end 120.65 85.6996) (width 0.3) (layer "B.Cu") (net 12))
 (segment (start 120.65 85.6996) (end 120.65 88.9) (width 0.3) (layer "B.Cu") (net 12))
 (segment (start 116.8908 83.3628) (end 118.3132 83.3628) (width 0.3) (layer "B.Cu") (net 12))
 (segment (start 125.6792 86.1314) (end 121.3104 86.1314) (width 0.3) (layer "F.Cu") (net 3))
 (segment (start 126.4158 85.1662) (end 126.4158 85.3948) (width 0.3) (layer "F.Cu") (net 3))
 (segment (start 126.4158 85.3948) (end 125.6792 86.1314) (width 0.3) (layer "F.Cu") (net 3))
 (segment (start 121.3104 86.1314) (end 120.65 86.7918) (width 0.3) (layer "F.Cu") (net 3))
 (segment (start 120.65 86.7918) (end 120.65 88.9) (width 0.3) (layer "F.Cu") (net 3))
 (via (at 126.4158 85.1662) (size 0.6) (drill 0.4) (layers "F.Cu" "B.Cu") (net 3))
 (segment (start 125.1204 77.6224) (end 124.6632 77.1652) (width 0.3) (layer "B.Cu") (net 3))
 (segment (start 125.1204 83.8708) (end 125.1204 77.6224) (width 0.3) (layer "B.Cu") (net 3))
 (segment (start 124.6632 77.1652) (end 122.4548 77.1652) (width 0.3) (layer "B.Cu") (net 3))
 (segment (start 122.4548 77.1652) (end 120.84 78.78) (width 0.3) (layer "B.Cu") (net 3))
 (segment (start 126.4158 85.1662) (end 125.1204 83.8708) (width 0.3) (layer "B.Cu") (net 3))
 (segment (start 123.19 88.9) (end 123.19 86.36) (width 0.3) (layer "B.Cu") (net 6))
 (segment (start 120.84 84.01) (end 120.84 81.28) (width 0.3) (layer "B.Cu") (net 6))
 (segment (start 123.19 86.36) (end 120.84 84.01) (width 0.3) (layer "B.Cu") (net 6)))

